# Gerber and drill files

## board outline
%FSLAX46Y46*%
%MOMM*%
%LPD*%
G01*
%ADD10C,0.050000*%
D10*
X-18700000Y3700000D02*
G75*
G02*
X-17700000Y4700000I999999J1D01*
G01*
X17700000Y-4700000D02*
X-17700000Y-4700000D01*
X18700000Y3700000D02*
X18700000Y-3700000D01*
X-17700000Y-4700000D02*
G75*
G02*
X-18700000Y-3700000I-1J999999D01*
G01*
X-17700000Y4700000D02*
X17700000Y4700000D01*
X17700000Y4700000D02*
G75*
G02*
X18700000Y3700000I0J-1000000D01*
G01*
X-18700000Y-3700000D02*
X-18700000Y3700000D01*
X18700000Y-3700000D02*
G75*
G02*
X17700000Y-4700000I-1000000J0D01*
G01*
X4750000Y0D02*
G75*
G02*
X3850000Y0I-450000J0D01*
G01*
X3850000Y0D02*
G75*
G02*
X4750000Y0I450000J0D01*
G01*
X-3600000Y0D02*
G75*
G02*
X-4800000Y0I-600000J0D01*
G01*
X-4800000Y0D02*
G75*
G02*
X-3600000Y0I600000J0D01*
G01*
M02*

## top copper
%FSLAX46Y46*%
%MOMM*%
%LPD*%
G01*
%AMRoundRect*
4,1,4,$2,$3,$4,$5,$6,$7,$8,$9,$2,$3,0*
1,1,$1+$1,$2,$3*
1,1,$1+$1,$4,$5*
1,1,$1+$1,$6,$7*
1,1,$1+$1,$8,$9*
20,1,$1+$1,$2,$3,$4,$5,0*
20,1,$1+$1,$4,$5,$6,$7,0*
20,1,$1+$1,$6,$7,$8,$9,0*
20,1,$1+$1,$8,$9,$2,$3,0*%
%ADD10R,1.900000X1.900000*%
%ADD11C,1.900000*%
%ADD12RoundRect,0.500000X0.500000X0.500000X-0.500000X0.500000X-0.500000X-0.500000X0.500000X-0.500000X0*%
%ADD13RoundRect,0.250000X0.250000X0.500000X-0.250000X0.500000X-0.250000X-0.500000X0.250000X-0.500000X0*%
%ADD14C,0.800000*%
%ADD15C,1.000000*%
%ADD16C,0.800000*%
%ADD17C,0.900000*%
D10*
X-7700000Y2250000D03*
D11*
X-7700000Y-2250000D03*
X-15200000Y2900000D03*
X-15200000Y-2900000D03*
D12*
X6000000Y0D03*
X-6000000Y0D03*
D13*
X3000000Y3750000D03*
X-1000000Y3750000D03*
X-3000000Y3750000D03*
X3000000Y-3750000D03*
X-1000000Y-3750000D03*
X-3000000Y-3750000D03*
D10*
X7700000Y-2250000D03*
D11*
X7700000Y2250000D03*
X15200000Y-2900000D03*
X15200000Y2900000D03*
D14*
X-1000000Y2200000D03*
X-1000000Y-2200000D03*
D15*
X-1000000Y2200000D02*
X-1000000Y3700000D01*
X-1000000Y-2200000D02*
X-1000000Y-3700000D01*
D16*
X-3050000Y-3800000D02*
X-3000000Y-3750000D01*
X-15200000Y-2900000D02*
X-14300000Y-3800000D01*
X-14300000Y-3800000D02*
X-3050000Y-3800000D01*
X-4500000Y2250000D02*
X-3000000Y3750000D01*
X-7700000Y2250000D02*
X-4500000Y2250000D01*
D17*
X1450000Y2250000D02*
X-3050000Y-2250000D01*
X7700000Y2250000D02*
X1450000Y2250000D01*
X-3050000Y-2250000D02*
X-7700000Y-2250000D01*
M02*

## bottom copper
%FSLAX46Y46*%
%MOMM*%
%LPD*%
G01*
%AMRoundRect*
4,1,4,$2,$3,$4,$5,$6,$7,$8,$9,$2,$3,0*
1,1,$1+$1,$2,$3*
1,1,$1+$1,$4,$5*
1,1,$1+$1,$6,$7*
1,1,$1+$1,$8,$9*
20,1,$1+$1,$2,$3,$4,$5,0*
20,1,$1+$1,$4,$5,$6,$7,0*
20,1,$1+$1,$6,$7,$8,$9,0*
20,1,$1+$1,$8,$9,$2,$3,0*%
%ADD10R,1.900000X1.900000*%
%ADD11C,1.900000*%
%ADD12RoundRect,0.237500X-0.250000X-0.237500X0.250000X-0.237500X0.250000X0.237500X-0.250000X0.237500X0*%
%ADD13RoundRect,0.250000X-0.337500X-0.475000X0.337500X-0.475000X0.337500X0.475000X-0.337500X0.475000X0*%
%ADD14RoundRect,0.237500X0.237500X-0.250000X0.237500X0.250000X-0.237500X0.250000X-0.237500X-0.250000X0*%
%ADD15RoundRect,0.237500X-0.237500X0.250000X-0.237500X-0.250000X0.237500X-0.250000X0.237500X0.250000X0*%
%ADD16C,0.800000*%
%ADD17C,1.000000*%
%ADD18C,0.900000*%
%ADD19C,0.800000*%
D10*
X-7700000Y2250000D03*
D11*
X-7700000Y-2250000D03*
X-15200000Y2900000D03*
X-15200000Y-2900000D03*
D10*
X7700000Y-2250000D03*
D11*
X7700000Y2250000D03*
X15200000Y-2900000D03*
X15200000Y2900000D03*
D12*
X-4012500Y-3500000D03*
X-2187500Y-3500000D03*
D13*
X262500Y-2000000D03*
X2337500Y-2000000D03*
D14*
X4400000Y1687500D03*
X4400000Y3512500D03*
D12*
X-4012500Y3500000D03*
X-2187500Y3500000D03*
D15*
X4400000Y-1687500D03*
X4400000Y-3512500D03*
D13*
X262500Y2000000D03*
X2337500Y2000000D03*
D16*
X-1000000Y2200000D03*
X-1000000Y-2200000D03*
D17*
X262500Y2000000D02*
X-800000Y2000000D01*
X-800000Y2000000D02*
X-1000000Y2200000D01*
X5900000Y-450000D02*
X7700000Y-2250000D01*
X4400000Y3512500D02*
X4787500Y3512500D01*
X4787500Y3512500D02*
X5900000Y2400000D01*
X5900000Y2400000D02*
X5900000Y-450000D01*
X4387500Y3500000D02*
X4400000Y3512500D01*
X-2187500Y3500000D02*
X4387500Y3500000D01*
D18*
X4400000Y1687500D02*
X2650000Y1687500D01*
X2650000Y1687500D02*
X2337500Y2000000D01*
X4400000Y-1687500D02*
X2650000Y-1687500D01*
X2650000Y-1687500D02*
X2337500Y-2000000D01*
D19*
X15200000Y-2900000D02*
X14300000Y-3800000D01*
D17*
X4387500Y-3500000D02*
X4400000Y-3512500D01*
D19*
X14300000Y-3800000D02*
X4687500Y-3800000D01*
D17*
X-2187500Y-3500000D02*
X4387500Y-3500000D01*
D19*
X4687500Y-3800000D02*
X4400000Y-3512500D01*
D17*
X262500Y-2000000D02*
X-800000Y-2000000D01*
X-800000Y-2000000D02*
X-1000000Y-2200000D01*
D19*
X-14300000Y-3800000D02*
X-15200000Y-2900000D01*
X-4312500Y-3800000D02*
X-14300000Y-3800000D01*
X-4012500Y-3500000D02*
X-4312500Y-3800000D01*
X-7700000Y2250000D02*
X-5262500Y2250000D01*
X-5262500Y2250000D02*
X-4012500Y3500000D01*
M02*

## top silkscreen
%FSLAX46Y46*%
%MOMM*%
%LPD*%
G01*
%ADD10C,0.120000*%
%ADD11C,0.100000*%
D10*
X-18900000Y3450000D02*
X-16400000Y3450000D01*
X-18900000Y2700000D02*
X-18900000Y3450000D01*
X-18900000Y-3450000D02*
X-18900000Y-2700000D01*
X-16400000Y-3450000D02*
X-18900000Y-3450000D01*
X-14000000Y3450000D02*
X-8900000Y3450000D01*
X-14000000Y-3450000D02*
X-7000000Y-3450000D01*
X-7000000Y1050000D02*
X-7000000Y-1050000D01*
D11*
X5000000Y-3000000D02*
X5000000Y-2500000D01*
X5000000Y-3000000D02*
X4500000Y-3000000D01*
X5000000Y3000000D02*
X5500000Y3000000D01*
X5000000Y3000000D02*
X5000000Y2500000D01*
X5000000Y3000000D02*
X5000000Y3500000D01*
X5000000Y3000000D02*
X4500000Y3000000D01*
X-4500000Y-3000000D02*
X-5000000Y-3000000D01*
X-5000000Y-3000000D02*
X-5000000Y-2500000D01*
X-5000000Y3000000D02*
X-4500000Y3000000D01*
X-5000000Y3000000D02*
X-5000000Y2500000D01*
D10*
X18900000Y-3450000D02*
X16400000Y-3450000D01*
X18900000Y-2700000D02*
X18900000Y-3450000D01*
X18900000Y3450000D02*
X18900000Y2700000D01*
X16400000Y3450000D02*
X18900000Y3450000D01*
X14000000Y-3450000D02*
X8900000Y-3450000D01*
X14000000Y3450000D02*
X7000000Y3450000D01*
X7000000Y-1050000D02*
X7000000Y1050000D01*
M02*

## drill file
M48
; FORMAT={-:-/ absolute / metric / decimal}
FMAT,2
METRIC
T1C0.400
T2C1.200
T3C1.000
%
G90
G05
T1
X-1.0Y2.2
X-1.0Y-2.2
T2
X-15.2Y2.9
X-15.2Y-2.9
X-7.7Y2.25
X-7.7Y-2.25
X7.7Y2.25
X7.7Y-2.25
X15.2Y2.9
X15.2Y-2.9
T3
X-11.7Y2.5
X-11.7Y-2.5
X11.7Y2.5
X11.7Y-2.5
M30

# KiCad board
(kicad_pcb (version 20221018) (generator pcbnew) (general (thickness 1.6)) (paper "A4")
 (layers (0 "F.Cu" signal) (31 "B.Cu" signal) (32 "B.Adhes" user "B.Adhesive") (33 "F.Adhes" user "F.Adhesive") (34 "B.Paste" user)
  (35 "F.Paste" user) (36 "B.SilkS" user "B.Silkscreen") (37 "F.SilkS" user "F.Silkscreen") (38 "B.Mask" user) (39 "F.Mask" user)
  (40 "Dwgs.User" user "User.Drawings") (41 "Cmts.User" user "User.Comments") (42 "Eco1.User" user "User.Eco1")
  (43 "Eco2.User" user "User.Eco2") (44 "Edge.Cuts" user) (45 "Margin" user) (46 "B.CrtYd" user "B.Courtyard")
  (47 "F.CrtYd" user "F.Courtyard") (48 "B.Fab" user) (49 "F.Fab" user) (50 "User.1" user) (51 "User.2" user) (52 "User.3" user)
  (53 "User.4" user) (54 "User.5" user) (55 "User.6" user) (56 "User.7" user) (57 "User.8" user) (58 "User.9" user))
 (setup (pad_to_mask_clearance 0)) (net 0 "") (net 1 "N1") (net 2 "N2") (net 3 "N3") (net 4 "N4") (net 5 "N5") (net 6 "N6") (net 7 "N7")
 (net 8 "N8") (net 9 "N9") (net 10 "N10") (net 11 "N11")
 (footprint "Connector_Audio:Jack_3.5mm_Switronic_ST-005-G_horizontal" (layer "F.Cu") (at -14.2 0)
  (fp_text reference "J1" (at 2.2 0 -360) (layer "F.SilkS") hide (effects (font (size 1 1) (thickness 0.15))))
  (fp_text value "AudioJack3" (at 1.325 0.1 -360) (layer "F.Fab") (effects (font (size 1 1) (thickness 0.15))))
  (fp_line (start -4.7 -3.45) (end -2.2 -3.45) (stroke (width 0.12) (type solid)) (layer "F.SilkS"))
  (fp_line (start -4.7 -2.7) (end -4.7 -3.45) (stroke (width 0.12) (type solid)) (layer "F.SilkS"))
  (fp_line (start -4.7 3.45) (end -4.7 2.7) (stroke (width 0.12) (type solid)) (layer "F.SilkS"))
  (fp_line (start -2.2 3.45) (end -4.7 3.45) (stroke (width 0.12) (type solid)) (layer "F.SilkS"))
  (fp_line (start 0.2 -3.45) (end 5.3 -3.45) (stroke (width 0.12) (type solid)) (layer "F.SilkS"))
  (fp_line (start 0.2 3.45) (end 7.2 3.45) (stroke (width 0.12) (type solid)) (layer "F.SilkS"))
  (fp_line (start 7.2 -1.05) (end 7.2 1.05) (stroke (width 0.12) (type solid)) (layer "F.SilkS"))
  (pad "" np_thru_hole circle (at 2.5 -2.5) (size 1 1) (drill 1) (layers "*.Cu" "*.Mask"))
  (pad "" np_thru_hole circle (at 2.5 2.5) (size 1 1) (drill 1) (layers "*.Cu" "*.Mask"))
  (pad "R" thru_hole rect (at 6.5 -2.25) (size 1.9 1.9) (drill 1.2) (layers "*.Cu" "*.Mask") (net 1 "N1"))
  (pad "S" thru_hole circle (at 6.5 2.25) (size 1.9 1.9) (drill 1.2) (layers "*.Cu" "*.Mask") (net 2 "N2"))
  (pad "T" thru_hole circle (at -1 -2.9) (size 1.9 1.9) (drill 1.2) (layers "*.Cu" "*.Mask") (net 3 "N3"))
  (pad "T" thru_hole circle (at -1 2.9) (size 1.9 1.9) (drill 1.2) (layers "*.Cu" "*.Mask") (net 3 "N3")))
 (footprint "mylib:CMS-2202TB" (layer "F.Cu") (at 0 0 180)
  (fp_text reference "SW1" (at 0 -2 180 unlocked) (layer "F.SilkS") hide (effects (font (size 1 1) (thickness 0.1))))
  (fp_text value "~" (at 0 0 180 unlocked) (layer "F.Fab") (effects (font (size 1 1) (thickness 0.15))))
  (fp_line (start -5 -3) (end -5 -2.5) (stroke (width 0.1) (type default)) (layer "F.SilkS"))
  (fp_line (start -5 -3) (end -4.5 -3) (stroke (width 0.1) (type default)) (layer "F.SilkS"))
  (fp_line (start -5 3) (end -5.5 3) (stroke (width 0.1) (type default)) (layer "F.SilkS"))
  (fp_line (start -5 3) (end -5 2.5) (stroke (width 0.1) (type default)) (layer "F.SilkS"))
  (fp_line (start -5 3) (end -5 3.5) (stroke (width 0.1) (type default)) (layer "F.SilkS"))
  (fp_line (start -5 3) (end -4.5 3) (stroke (width 0.1) (type default)) (layer "F.SilkS"))
  (fp_line (start 4.5 -3) (end 5 -3) (stroke (width 0.1) (type default)) (layer "F.SilkS"))
  (fp_line (start 5 -3) (end 5 -2.5) (stroke (width 0.1) (type default)) (layer "F.SilkS"))
  (fp_line (start 5 3) (end 4.5 3) (stroke (width 0.1) (type default)) (layer "F.SilkS"))
  (fp_line (start 5 3) (end 5 2.5) (stroke (width 0.1) (type default)) (layer "F.SilkS"))
  (fp_circle (center -4.3 0) (end -3.85 0) (stroke (width 0.05) (type default)) (fill none) (layer "Edge.Cuts"))
  (fp_circle (center 4.2 0) (end 4.8 0) (stroke (width 0.05) (type default)) (fill none) (layer "Edge.Cuts"))
  (pad "" smd roundrect (at -6 0 180) (size 2 2) (layers "F.Cu" "F.Paste" "F.Mask") (roundrect_rratio 0.25) (thermal_bridge_angle 45))
  (pad "" smd roundrect (at 6 0 180) (size 2 2) (layers "F.Cu" "F.Paste" "F.Mask") (roundrect_rratio 0.25) (thermal_bridge_angle 45))
  (pad "1" smd roundrect (at -3 3.75 180) (size 1 1.5) (layers "F.Cu" "F.Paste" "F.Mask") (roundrect_rratio 0.25) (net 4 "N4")
   (thermal_bridge_angle 45))
  (pad "2" smd roundrect (at 1 3.75 180) (size 1 1.5) (layers "F.Cu" "F.Paste" "F.Mask") (roundrect_rratio 0.25) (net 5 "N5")
   (thermal_bridge_angle 45))
  (pad "3" smd roundrect (at 3 3.75 180) (size 1 1.5) (layers "F.Cu" "F.Paste" "F.Mask") (roundrect_rratio 0.25) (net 1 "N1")
   (thermal_bridge_angle 45))
  (pad "4" smd roundrect (at -3 -3.75 180) (size 1 1.5) (layers "F.Cu" "F.Paste" "F.Mask") (roundrect_rratio 0.25) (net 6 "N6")
   (thermal_bridge_angle 45))
  (pad "5" smd roundrect (at 1 -3.75 180) (size 1 1.5) (layers "F.Cu" "F.Paste" "F.Mask") (roundrect_rratio 0.25) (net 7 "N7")
   (thermal_bridge_angle 45))
  (pad "6" smd roundrect (at 3 -3.75 180) (size 1 1.5) (layers "F.Cu" "F.Paste" "F.Mask") (roundrect_rratio 0.25) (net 3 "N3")
   (thermal_bridge_angle 45)))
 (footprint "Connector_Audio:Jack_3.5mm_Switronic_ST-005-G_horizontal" (layer "F.Cu") (at 14.2 0 180)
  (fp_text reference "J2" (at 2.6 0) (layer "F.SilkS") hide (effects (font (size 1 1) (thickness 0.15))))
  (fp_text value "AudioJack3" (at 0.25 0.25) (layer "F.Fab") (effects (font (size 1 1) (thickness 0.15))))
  (fp_line (start -4.7 -3.45) (end -2.2 -3.45) (stroke (width 0.12) (type solid)) (layer "F.SilkS"))
  (fp_line (start -4.7 -2.7) (end -4.7 -3.45) (stroke (width 0.12) (type solid)) (layer "F.SilkS"))
  (fp_line (start -4.7 3.45) (end -4.7 2.7) (stroke (width 0.12) (type solid)) (layer "F.SilkS"))
  (fp_line (start -2.2 3.45) (end -4.7 3.45) (stroke (width 0.12) (type solid)) (layer "F.SilkS"))
  (fp_line (start 0.2 -3.45) (end 5.3 -3.45) (stroke (width 0.12) (type solid)) (layer "F.SilkS"))
  (fp_line (start 0.2 3.45) (end 7.2 3.45) (stroke (width 0.12) (type solid)) (layer "F.SilkS"))
  (fp_line (start 7.2 -1.05) (end 7.2 1.05) (stroke (width 0.12) (type solid)) (layer "F.SilkS"))
  (pad "" np_thru_hole circle (at 2.5 -2.5 180) (size 1 1) (drill 1) (layers "*.Cu" "*.Mask"))
  (pad "" np_thru_hole circle (at 2.5 2.5 180) (size 1 1) (drill 1) (layers "*.Cu" "*.Mask"))
  (pad "R" thru_hole rect (at 6.5 -2.25 180) (size 1.9 1.9) (drill 1.2) (layers "*.Cu" "*.Mask") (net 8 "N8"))
  (pad "S" thru_hole circle (at 6.5 2.25 180) (size 1.9 1.9) (drill 1.2) (layers "*.Cu" "*.Mask") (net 2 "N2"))
  (pad "T" thru_hole circle (at -1 -2.9 180) (size 1.9 1.9) (drill 1.2) (layers "*.Cu" "*.Mask") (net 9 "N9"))
  (pad "T" thru_hole circle (at -1 2.9 180) (size 1.9 1.9) (drill 1.2) (layers "*.Cu" "*.Mask") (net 9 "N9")))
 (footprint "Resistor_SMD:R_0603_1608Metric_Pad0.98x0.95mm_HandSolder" (layer "B.Cu") (at -3.1 3.5)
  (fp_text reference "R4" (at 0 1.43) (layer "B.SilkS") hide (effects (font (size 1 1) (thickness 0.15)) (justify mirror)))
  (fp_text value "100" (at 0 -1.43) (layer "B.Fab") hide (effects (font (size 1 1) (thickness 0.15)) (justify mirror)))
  (pad "1" smd roundrect (at -0.9125 0) (size 0.975 0.95) (layers "B.Cu" "B.Paste" "B.Mask") (roundrect_rratio 0.25) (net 3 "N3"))
  (pad "2" smd roundrect (at 0.9125 0) (size 0.975 0.95) (layers "B.Cu" "B.Paste" "B.Mask") (roundrect_rratio 0.25) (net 9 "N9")))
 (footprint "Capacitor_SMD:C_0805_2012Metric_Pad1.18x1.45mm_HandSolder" (layer "B.Cu") (at 1.3 2)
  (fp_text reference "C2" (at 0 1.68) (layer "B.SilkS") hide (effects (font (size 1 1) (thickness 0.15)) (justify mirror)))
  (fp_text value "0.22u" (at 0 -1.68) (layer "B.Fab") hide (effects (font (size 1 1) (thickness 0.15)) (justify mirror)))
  (pad "1" smd roundrect (at -1.0375 0) (size 1.175 1.45) (layers "B.Cu" "B.Paste" "B.Mask") (roundrect_rratio 0.2127659574) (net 7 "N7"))
  (pad "2" smd roundrect (at 1.0375 0) (size 1.175 1.45) (layers "B.Cu" "B.Paste" "B.Mask") (roundrect_rratio 0.2127659574) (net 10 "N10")))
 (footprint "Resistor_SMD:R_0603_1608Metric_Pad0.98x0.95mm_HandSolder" (layer "B.Cu") (at 4.4 -2.6 90)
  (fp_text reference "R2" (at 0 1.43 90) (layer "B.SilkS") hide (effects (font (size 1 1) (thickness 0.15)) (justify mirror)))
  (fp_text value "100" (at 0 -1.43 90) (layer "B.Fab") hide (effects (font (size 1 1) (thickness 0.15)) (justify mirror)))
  (pad "1" smd roundrect (at -0.9125 0 90) (size 0.975 0.95) (layers "B.Cu" "B.Paste" "B.Mask") (roundrect_rratio 0.25) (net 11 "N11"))
  (pad "2" smd roundrect (at 0.9125 0 90) (size 0.975 0.95) (layers "B.Cu" "B.Paste" "B.Mask") (roundrect_rratio 0.25) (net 8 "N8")))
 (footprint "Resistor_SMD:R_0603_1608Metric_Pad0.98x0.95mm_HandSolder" (layer "B.Cu") (at -3.1 -3.5)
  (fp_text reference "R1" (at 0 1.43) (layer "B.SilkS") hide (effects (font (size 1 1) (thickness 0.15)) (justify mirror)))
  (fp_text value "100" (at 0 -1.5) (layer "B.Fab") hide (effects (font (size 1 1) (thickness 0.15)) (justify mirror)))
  (pad "1" smd roundrect (at -0.9125 0) (size 0.975 0.95) (layers "B.Cu" "B.Paste" "B.Mask") (roundrect_rratio 0.25) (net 1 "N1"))
  (pad "2" smd roundrect (at 0.9125 0) (size 0.975 0.95) (layers "B.Cu" "B.Paste" "B.Mask") (roundrect_rratio 0.25) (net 8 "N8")))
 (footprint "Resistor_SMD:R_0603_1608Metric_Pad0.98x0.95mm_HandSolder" (layer "B.Cu") (at 4.4 2.6 -90)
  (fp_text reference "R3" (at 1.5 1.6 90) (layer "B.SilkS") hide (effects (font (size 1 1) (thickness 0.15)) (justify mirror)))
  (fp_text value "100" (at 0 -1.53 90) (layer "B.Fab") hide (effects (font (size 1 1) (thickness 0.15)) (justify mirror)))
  (pad "1" smd roundrect (at -0.9125 0 270) (size 0.975 0.95) (layers "B.Cu" "B.Paste" "B.Mask") (roundrect_rratio 0.25) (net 10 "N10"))
  (pad "2" smd roundrect (at 0.9125 0 270) (size 0.975 0.95) (layers "B.Cu" "B.Paste" "B.Mask") (roundrect_rratio 0.25) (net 9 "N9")))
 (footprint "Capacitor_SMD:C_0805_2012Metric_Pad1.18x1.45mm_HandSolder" (layer "B.Cu") (at 1.3 -2)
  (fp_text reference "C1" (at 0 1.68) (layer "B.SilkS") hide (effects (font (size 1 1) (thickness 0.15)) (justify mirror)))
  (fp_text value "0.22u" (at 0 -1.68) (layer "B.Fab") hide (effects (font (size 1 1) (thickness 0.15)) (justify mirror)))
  (pad "1" smd roundrect (at -1.0375 0) (size 1.175 1.45) (layers "B.Cu" "B.Paste" "B.Mask") (roundrect_rratio 0.2127659574) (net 5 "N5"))
  (pad "2" smd roundrect (at 1.0375 0) (size 1.175 1.45) (layers "B.Cu" "B.Paste" "B.Mask") (roundrect_rratio 0.2127659574) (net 11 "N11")))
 (gr_arc (start -18.7 -3.7) (mid -18.407107 -4.407107) (end -17.7 -4.7) (stroke (width 0.05) (type default)) (layer "Edge.Cuts"))
 (gr_line (start 17.7 4.7) (end -17.7 4.7) (stroke (width 0.05) (type default)) (layer "Edge.Cuts"))
 (gr_line (start 18.7 -3.7) (end 18.7 3.7) (stroke (width 0.05) (type default)) (layer "Edge.Cuts"))
 (gr_arc (start -17.7 4.7) (mid -18.407107 4.407107) (end -18.7 3.7) (stroke (width 0.05) (type default)) (layer "Edge.Cuts"))
 (gr_line (start -17.7 -4.7) (end 17.7 -4.7) (stroke (width 0.05) (type default)) (layer "Edge.Cuts"))
 (gr_arc (start 17.7 -4.7) (mid 18.407107 -4.407107) (end 18.7 -3.7) (stroke (width 0.05) (type default)) (layer "Edge.Cuts"))
 (gr_line (start -18.7 3.7) (end -18.7 -3.7) (stroke (width 0.05) (type default)) (layer "Edge.Cuts"))
 (gr_arc (start 18.7 3.7) (mid 18.407107 4.407107) (end 17.7 4.7) (stroke (width 0.05) (type default)) (layer "Edge.Cuts"))
 (segment (start -1 -2.2) (end -1 -3.7) (width 1) (layer "F.Cu") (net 5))
 (via (at -1 -2.2) (size 0.8) (drill 0.4) (layers "F.Cu" "B.Cu") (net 5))
 (segment (start 0.2625 -2) (end -0.8 -2) (width 1) (layer "B.Cu") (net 5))
 (segment (start -0.8 -2) (end -1 -2.2) (width 1) (layer "B.Cu") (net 5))
 (segment (start 5.9 0.45) (end 7.7 2.25) (width 1) (layer "B.Cu") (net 8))
 (segment (start 4.4 -3.5125) (end 4.7875 -3.5125) (width 1) (layer "B.Cu") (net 8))
 (segment (start 4.7875 -3.5125) (end 5.9 -2.4) (width 1) (layer "B.Cu") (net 8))
 (segment (start 5.9 -2.4) (end 5.9 0.45) (width 1) (layer "B.Cu") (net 8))
 (segment (start 4.3875 -3.5) (end 4.4 -3.5125) (width 1) (layer "B.Cu") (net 8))
 (segment (start -2.1875 -3.5) (end 4.3875 -3.5) (width 1) (layer "B.Cu") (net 8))
 (segment (start 4.4 -1.6875) (end 2.65 -1.6875) (width 0.9) (layer "B.Cu") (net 11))
 (segment (start 2.65 -1.6875) (end 2.3375 -2) (width 0.9) (layer "B.Cu") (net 11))
 (segment (start 4.4 1.6875) (end 2.65 1.6875) (width 0.9) (layer "B.Cu") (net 10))
 (segment (start 2.65 1.6875) (end 2.3375 2) (width 0.9) (layer "B.Cu") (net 10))
 (segment (start 15.2 2.9) (end 14.3 3.8) (width 0.8) (layer "B.Cu") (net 9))
 (segment (start 4.3875 3.5) (end 4.4 3.5125) (width 1) (layer "B.Cu") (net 9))
 (segment (start 14.3 3.8) (end 4.6875 3.8) (width 0.8) (layer "B.Cu") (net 9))
 (segment (start -2.1875 3.5) (end 4.3875 3.5) (width 1) (layer "B.Cu") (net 9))
 (segment (start 4.6875 3.8) (end 4.4 3.5125) (width 0.8) (layer "B.Cu") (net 9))
 (segment (start -1 2.2) (end -1 3.7) (width 1) (layer "F.Cu") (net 7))
 (via (at -1 2.2) (size 0.8) (drill 0.4) (layers "F.Cu" "B.Cu") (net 7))
 (segment (start 0.2625 2) (end -0.8 2) (width 1) (layer "B.Cu") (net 7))
 (segment (start -0.8 2) (end -1 2.2) (width 1) (layer "B.Cu") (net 7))
 (segment (start -3.05 3.8) (end -3 3.75) (width 0.8) (layer "F.Cu") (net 3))
 (segment (start -15.2 2.9) (end -14.3 3.8) (width 0.8) (layer "F.Cu") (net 3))
 (segment (start -14.3 3.8) (end -3.05 3.8) (width 0.8) (layer "F.Cu") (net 3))
 (segment (start -14.3 3.8) (end -15.2 2.9) (width 0.8) (layer "B.Cu") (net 3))
 (segment (start -4.3125 3.8) (end -14.3 3.8) (width 0.8) (layer "B.Cu") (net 3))
 (segment (start -4.0125 3.5) (end -4.3125 3.8) (width 0.8) (layer "B.Cu") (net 3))
 (segment (start -4.5 -2.25) (end -3 -3.75) (width 0.8) (layer "F.Cu") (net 1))
 (segment (start -7.7 -2.25) (end -4.5 -2.25) (width 0.8) (layer "F.Cu") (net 1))
 (segment (start -7.7 -2.25) (end -5.2625 -2.25) (width 0.8) (layer "B.Cu") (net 1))
 (segment (start -5.2625 -2.25) (end -4.0125 -3.5) (width 0.8) (layer "B.Cu") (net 1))
 (segment (start 1.45 -2.25) (end -3.05 2.25) (width 0.9) (layer "F.Cu") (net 2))
 (segment (start 7.7 -2.25) (end 1.45 -2.25) (width 0.9) (layer "F.Cu") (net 2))
 (segment (start -3.05 2.25) (end -7.7 2.25) (width 0.9) (layer "F.Cu") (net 2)))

